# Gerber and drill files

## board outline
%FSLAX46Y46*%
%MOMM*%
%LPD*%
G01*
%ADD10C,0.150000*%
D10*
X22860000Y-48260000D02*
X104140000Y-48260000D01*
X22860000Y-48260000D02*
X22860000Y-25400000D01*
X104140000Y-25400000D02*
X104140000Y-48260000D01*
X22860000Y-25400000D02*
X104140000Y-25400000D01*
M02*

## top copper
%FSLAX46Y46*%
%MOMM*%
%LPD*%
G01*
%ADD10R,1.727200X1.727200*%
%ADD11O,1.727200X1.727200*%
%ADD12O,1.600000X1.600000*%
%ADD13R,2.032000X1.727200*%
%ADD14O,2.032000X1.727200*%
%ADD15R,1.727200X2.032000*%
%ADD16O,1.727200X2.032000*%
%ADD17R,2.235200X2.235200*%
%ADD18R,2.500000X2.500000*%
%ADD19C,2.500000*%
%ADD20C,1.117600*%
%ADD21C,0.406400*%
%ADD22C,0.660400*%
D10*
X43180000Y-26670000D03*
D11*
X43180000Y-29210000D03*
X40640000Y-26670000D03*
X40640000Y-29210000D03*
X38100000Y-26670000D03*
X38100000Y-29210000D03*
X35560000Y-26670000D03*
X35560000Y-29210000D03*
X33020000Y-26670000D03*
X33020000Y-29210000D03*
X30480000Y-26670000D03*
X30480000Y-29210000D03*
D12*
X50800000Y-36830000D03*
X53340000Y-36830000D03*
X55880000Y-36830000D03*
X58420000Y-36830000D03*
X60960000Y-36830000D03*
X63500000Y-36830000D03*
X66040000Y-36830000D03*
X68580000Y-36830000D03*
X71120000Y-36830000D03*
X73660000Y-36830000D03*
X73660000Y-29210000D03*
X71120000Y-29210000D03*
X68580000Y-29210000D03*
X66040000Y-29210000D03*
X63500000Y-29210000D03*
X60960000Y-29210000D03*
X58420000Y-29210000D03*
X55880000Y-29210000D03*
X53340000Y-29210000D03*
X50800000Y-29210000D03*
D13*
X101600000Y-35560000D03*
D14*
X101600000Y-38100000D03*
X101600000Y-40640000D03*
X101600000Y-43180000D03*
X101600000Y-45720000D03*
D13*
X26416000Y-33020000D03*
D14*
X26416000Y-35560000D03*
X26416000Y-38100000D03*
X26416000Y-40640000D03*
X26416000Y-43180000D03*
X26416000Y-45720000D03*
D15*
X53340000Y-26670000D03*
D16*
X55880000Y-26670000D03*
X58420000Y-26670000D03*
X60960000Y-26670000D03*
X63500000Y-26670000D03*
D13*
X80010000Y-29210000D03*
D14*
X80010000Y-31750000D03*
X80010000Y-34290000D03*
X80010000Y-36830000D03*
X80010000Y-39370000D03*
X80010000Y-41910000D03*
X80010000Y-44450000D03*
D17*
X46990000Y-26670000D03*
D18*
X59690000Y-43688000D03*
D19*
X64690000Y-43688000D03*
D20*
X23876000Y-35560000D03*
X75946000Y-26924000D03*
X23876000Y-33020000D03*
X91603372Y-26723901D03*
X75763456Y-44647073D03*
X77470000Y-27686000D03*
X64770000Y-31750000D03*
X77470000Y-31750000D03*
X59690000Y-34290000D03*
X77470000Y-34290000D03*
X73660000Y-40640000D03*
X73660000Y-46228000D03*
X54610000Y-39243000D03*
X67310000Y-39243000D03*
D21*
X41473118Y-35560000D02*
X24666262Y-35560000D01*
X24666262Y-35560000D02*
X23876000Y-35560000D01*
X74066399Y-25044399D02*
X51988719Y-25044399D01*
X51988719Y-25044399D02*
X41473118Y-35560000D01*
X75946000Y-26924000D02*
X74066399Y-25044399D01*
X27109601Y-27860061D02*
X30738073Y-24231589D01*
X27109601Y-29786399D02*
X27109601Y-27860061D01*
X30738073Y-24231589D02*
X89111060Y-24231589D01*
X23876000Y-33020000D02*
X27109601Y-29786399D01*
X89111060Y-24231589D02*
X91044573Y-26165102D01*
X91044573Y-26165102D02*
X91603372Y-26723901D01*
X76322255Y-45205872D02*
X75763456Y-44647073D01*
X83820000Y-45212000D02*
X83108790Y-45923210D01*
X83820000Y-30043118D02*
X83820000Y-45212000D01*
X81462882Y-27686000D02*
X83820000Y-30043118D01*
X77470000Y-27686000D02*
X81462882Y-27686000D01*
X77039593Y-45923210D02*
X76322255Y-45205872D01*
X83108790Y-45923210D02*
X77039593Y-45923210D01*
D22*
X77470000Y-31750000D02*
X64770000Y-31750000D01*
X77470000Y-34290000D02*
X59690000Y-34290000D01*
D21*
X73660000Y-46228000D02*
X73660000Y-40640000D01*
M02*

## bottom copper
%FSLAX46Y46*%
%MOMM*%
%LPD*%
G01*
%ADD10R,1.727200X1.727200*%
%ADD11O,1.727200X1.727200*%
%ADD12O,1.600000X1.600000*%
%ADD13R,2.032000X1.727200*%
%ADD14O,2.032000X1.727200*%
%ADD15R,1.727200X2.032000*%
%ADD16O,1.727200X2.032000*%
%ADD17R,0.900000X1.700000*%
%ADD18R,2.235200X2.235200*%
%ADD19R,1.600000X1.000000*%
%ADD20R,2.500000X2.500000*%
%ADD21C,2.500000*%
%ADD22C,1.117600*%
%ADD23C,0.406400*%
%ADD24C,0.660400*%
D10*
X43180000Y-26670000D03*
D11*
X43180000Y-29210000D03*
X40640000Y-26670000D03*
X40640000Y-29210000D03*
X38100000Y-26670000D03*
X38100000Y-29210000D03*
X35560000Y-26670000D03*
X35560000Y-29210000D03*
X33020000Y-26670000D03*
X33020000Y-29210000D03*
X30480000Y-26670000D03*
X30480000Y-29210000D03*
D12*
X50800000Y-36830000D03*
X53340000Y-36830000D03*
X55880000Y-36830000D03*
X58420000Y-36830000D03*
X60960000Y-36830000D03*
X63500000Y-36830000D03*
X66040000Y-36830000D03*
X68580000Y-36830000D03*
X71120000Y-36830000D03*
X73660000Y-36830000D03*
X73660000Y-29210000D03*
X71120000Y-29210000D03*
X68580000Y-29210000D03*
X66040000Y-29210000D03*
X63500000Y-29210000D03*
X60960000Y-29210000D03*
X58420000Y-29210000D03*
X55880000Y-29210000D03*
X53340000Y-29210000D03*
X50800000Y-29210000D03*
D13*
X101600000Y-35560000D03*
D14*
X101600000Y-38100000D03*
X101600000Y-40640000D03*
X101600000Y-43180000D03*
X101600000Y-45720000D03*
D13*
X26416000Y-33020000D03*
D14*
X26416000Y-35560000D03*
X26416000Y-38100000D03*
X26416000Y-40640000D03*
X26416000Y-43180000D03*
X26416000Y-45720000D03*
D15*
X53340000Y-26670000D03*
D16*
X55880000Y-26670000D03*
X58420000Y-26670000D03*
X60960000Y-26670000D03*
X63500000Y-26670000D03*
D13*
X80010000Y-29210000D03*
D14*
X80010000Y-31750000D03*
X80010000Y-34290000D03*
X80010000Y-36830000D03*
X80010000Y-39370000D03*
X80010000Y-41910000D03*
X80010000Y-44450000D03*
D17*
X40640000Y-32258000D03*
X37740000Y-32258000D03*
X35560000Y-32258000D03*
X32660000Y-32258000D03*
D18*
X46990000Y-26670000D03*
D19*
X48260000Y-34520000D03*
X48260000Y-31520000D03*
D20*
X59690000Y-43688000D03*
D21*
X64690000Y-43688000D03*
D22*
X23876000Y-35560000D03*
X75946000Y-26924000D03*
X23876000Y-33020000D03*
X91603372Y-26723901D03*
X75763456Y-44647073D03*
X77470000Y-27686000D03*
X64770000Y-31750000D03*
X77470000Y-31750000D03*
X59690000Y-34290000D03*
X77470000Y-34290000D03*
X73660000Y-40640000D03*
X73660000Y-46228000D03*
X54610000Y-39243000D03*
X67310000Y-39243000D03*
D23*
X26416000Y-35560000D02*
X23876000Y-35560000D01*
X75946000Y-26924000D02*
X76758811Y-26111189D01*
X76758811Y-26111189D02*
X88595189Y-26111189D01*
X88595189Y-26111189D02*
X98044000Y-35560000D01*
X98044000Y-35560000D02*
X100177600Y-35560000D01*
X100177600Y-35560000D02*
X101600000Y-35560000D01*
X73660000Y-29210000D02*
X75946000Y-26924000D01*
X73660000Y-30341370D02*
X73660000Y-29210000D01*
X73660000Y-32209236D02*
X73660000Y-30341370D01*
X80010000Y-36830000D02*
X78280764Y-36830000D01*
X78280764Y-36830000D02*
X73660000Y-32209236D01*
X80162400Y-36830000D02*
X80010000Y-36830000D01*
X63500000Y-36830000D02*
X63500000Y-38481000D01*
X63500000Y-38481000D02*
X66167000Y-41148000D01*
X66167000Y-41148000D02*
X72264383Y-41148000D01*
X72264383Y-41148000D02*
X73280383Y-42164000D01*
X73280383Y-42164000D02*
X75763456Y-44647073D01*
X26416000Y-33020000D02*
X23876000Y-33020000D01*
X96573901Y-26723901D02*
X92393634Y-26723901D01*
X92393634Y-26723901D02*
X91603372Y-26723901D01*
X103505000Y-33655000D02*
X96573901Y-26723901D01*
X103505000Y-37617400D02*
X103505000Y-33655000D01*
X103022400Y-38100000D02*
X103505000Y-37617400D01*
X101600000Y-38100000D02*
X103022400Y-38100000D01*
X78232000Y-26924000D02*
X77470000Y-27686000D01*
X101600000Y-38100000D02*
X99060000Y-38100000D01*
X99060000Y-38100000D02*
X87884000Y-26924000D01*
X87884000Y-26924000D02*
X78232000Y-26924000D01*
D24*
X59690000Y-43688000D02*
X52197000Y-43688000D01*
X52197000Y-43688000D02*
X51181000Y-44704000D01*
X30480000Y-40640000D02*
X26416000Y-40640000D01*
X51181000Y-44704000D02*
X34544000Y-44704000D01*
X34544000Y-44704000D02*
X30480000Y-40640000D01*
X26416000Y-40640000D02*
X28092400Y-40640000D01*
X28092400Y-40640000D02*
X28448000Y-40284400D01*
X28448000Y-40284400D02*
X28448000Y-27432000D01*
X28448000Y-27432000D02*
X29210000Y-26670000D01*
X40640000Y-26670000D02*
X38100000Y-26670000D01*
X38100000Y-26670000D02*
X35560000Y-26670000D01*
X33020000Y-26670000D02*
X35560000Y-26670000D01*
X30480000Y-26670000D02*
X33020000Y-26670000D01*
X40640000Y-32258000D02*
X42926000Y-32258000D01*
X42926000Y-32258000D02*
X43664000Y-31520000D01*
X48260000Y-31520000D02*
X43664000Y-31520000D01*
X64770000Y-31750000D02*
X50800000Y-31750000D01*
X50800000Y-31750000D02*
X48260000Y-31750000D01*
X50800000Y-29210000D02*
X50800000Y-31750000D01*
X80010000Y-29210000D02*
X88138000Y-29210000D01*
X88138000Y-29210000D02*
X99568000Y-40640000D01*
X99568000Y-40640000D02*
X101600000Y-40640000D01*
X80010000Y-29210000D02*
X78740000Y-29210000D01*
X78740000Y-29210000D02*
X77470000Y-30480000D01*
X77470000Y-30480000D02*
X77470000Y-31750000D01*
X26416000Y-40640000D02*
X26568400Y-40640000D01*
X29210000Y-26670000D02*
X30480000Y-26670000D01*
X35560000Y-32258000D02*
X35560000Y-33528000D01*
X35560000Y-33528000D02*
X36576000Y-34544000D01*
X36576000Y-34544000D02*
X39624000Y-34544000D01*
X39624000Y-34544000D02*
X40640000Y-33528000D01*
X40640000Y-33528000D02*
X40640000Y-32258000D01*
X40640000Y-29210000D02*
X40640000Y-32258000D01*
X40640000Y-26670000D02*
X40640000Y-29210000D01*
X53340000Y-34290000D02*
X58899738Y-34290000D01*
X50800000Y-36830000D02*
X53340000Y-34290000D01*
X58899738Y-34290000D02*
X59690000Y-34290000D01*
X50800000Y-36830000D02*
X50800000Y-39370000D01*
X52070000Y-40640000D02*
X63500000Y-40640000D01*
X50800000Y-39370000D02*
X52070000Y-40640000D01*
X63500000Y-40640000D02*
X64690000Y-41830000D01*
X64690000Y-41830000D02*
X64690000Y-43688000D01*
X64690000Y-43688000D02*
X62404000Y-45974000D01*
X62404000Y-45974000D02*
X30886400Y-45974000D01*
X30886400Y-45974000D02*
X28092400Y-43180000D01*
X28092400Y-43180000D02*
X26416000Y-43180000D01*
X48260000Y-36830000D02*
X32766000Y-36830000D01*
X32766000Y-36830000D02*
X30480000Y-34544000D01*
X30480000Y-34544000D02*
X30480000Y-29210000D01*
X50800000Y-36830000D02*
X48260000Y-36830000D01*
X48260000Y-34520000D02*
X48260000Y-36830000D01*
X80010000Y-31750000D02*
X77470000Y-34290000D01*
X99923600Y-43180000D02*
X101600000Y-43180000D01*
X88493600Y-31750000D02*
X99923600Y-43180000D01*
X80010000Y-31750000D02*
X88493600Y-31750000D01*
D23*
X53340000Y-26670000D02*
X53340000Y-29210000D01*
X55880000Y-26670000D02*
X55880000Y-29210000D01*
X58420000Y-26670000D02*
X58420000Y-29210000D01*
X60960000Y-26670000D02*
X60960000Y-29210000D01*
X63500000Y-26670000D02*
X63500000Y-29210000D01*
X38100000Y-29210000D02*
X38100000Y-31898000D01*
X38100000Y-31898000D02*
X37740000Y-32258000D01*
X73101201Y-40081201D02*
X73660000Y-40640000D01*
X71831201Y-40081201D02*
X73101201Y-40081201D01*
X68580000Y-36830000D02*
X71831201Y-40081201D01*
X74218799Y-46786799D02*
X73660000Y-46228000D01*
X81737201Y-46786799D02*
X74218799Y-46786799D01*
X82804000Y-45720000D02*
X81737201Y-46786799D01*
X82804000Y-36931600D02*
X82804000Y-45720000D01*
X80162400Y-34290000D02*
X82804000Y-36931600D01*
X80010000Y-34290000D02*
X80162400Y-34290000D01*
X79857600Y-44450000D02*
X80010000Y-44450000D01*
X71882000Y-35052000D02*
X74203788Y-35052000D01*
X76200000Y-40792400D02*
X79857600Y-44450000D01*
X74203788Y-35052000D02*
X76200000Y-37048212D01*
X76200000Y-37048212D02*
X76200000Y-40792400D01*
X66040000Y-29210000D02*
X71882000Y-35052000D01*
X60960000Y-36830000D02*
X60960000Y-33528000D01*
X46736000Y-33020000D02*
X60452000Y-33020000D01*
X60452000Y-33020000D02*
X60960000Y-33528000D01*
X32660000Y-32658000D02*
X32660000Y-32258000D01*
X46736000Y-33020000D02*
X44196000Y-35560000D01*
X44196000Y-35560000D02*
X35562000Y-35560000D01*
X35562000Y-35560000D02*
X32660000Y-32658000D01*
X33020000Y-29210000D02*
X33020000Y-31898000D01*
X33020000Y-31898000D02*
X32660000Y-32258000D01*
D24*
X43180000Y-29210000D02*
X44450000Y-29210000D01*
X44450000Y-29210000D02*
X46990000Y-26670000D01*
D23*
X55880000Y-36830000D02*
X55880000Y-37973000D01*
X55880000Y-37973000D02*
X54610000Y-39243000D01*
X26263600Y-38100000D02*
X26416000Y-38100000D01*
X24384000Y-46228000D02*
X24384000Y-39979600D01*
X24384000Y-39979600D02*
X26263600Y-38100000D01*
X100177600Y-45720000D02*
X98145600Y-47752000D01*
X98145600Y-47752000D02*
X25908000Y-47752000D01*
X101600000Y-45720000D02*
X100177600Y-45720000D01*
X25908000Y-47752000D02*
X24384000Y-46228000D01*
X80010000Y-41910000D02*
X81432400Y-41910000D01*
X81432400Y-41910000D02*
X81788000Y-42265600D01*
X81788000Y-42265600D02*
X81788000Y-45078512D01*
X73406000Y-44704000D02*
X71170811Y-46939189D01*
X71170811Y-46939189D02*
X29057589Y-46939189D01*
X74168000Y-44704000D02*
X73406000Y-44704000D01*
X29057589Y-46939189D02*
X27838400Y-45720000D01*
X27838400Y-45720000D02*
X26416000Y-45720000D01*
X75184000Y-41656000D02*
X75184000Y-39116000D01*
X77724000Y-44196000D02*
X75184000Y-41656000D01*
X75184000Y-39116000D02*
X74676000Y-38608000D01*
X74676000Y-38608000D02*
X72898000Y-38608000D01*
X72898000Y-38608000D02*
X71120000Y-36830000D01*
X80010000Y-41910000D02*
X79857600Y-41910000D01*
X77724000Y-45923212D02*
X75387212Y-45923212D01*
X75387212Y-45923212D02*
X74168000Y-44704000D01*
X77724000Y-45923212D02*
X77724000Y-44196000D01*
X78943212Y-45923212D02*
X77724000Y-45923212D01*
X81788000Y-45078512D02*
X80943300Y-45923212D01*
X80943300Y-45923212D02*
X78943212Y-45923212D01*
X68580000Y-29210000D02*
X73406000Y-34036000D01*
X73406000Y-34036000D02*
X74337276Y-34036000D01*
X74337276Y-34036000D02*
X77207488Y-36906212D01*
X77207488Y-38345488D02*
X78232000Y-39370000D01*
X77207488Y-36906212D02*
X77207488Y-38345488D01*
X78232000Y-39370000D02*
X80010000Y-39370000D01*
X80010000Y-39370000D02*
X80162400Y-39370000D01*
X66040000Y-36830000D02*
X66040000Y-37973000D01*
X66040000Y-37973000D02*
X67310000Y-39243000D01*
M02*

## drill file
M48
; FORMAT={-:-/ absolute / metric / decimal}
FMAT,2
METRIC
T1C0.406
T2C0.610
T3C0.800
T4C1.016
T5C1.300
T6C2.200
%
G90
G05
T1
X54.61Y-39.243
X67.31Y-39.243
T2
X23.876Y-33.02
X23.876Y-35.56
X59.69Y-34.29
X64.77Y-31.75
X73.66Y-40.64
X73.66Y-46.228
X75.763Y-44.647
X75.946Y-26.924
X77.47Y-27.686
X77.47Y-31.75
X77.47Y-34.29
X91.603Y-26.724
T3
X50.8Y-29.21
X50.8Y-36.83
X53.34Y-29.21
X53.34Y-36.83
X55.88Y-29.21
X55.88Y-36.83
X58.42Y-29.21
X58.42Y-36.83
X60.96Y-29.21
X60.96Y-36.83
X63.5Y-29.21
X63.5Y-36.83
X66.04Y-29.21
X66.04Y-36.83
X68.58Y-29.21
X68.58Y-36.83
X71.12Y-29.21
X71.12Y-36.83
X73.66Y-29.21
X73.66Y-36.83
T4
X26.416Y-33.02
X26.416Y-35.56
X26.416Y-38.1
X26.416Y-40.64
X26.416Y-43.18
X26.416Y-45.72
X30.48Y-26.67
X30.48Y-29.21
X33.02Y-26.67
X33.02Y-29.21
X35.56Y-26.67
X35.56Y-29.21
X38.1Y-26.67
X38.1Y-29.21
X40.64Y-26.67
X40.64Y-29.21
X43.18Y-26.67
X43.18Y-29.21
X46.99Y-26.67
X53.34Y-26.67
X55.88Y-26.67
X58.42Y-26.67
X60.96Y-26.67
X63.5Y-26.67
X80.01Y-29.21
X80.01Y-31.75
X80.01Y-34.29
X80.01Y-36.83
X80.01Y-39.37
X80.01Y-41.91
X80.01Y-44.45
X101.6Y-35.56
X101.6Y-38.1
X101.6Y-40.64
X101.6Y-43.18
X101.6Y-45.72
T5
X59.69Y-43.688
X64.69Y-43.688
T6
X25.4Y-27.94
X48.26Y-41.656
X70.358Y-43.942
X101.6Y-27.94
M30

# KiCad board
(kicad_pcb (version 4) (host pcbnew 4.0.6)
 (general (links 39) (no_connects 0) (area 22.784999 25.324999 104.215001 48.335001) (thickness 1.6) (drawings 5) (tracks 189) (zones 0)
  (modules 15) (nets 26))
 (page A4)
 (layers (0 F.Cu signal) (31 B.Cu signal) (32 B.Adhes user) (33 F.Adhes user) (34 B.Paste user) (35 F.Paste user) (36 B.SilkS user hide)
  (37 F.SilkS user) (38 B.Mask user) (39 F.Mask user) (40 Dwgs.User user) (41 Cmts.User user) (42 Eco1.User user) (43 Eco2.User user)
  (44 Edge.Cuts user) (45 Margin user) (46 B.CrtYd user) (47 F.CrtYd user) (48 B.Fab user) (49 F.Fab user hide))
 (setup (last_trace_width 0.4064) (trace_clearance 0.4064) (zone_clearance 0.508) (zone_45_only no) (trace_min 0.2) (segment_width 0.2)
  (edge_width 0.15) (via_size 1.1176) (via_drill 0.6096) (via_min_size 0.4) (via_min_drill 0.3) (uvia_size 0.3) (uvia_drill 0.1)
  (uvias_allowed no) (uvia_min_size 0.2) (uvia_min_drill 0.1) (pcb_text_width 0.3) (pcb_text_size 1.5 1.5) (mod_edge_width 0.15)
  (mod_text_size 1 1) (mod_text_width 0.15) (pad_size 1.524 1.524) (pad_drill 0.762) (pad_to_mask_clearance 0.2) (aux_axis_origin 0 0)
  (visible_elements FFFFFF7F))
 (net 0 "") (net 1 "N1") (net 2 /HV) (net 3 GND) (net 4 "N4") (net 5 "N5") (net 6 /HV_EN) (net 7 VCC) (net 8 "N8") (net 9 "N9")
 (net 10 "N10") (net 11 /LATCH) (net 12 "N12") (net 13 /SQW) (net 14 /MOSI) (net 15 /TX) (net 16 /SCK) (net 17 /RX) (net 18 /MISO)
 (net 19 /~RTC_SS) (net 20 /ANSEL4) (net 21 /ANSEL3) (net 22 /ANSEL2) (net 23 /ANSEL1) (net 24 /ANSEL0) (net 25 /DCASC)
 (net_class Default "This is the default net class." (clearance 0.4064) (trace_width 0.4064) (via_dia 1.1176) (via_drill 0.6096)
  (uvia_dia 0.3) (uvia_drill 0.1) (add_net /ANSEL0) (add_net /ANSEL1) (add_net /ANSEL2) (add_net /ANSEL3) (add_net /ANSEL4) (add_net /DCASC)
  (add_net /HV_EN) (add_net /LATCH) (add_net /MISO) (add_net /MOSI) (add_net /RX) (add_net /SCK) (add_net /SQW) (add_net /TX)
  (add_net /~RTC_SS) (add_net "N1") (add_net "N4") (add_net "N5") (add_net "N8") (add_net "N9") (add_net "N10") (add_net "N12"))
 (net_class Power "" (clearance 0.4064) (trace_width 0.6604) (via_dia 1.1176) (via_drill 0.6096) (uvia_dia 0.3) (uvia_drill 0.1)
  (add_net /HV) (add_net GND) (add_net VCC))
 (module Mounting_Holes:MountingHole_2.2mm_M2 (layer F.Cu) (at 70.358 43.942)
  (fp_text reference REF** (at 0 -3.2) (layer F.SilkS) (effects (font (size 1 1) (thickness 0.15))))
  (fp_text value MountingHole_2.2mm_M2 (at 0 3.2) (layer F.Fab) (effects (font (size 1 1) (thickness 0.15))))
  (pad 1 np_thru_hole circle (at 0 0) (size 2.2 2.2) (drill 2.2) (layers *.Cu *.Mask)))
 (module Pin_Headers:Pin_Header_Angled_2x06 (layer F.Cu) (at 43.18 26.67 270)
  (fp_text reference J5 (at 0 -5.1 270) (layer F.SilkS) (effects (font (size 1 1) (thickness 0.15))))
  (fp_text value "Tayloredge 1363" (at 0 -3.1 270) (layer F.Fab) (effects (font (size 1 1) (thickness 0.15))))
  (pad 1 thru_hole rect (at 0 0 270) (size 1.7272 1.7272) (drill 1.016) (layers *.Cu *.Mask) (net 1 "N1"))
  (pad 2 thru_hole oval (at 2.54 0 270) (size 1.7272 1.7272) (drill 1.016) (layers *.Cu *.Mask) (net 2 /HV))
  (pad 3 thru_hole oval (at 0 2.54 270) (size 1.7272 1.7272) (drill 1.016) (layers *.Cu *.Mask) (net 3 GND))
  (pad 4 thru_hole oval (at 2.54 2.54 270) (size 1.7272 1.7272) (drill 1.016) (layers *.Cu *.Mask) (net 3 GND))
  (pad 5 thru_hole oval (at 0 5.08 270) (size 1.7272 1.7272) (drill 1.016) (layers *.Cu *.Mask) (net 3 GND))
  (pad 6 thru_hole oval (at 2.54 5.08 270) (size 1.7272 1.7272) (drill 1.016) (layers *.Cu *.Mask) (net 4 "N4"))
  (pad 7 thru_hole oval (at 0 7.62 270) (size 1.7272 1.7272) (drill 1.016) (layers *.Cu *.Mask) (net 3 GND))
  (pad 8 thru_hole oval (at 2.54 7.62 270) (size 1.7272 1.7272) (drill 1.016) (layers *.Cu *.Mask) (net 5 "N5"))
  (pad 9 thru_hole oval (at 0 10.16 270) (size 1.7272 1.7272) (drill 1.016) (layers *.Cu *.Mask) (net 3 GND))
  (pad 10 thru_hole oval (at 2.54 10.16 270) (size 1.7272 1.7272) (drill 1.016) (layers *.Cu *.Mask) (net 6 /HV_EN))
  (pad 11 thru_hole oval (at 0 12.7 270) (size 1.7272 1.7272) (drill 1.016) (layers *.Cu *.Mask) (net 3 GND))
  (pad 12 thru_hole oval (at 2.54 12.7 270) (size 1.7272 1.7272) (drill 1.016) (layers *.Cu *.Mask) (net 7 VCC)))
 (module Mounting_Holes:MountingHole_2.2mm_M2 (layer F.Cu) (at 48.26 41.656)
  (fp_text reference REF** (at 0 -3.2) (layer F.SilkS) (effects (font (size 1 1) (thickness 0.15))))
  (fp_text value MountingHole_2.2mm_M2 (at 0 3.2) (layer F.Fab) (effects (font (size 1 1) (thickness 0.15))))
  (pad 1 np_thru_hole circle (at 0 0) (size 2.2 2.2) (drill 2.2) (layers *.Cu *.Mask)))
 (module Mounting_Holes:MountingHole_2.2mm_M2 (layer F.Cu) (at 25.4 27.94)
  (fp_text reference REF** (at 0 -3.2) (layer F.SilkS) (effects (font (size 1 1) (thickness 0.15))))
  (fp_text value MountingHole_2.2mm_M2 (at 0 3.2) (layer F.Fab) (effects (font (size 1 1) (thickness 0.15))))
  (pad 1 np_thru_hole circle (at 0 0) (size 2.2 2.2) (drill 2.2) (layers *.Cu *.Mask)))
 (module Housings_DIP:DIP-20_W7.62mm (layer F.Cu) (at 50.8 36.83 90)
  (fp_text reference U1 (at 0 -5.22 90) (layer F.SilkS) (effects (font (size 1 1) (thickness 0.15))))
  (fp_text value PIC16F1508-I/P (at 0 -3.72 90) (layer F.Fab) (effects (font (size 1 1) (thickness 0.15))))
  (pad 1 thru_hole oval (at 0 0 90) (size 1.6 1.6) (drill 0.8) (layers *.Cu *.Mask) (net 7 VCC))
  (pad 2 thru_hole oval (at 0 2.54 90) (size 1.6 1.6) (drill 0.8) (layers *.Cu *.Mask) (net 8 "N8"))
  (pad 3 thru_hole oval (at 0 5.08 90) (size 1.6 1.6) (drill 0.8) (layers *.Cu *.Mask) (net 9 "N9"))
  (pad 4 thru_hole oval (at 0 7.62 90) (size 1.6 1.6) (drill 0.8) (layers *.Cu *.Mask) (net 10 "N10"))
  (pad 5 thru_hole oval (at 0 10.16 90) (size 1.6 1.6) (drill 0.8) (layers *.Cu *.Mask) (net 6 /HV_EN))
  (pad 6 thru_hole oval (at 0 12.7 90) (size 1.6 1.6) (drill 0.8) (layers *.Cu *.Mask) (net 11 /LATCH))
  (pad 7 thru_hole oval (at 0 15.24 90) (size 1.6 1.6) (drill 0.8) (layers *.Cu *.Mask) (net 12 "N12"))
  (pad 8 thru_hole oval (at 0 17.78 90) (size 1.6 1.6) (drill 0.8) (layers *.Cu *.Mask) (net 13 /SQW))
  (pad 9 thru_hole oval (at 0 20.32 90) (size 1.6 1.6) (drill 0.8) (layers *.Cu *.Mask) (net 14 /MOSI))
  (pad 10 thru_hole oval (at 0 22.86 90) (size 1.6 1.6) (drill 0.8) (layers *.Cu *.Mask) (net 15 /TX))
  (pad 11 thru_hole oval (at 7.62 22.86 90) (size 1.6 1.6) (drill 0.8) (layers *.Cu *.Mask) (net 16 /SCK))
  (pad 12 thru_hole oval (at 7.62 20.32 90) (size 1.6 1.6) (drill 0.8) (layers *.Cu *.Mask) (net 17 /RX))
  (pad 13 thru_hole oval (at 7.62 17.78 90) (size 1.6 1.6) (drill 0.8) (layers *.Cu *.Mask) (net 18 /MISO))
  (pad 14 thru_hole oval (at 7.62 15.24 90) (size 1.6 1.6) (drill 0.8) (layers *.Cu *.Mask) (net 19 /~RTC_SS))
  (pad 15 thru_hole oval (at 7.62 12.7 90) (size 1.6 1.6) (drill 0.8) (layers *.Cu *.Mask) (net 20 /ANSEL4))
  (pad 16 thru_hole oval (at 7.62 10.16 90) (size 1.6 1.6) (drill 0.8) (layers *.Cu *.Mask) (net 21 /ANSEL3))
  (pad 17 thru_hole oval (at 7.62 7.62 90) (size 1.6 1.6) (drill 0.8) (layers *.Cu *.Mask) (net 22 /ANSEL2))
  (pad 18 thru_hole oval (at 7.62 5.08 90) (size 1.6 1.6) (drill 0.8) (layers *.Cu *.Mask) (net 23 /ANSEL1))
  (pad 19 thru_hole oval (at 7.62 2.54 90) (size 1.6 1.6) (drill 0.8) (layers *.Cu *.Mask) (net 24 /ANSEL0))
  (pad 20 thru_hole oval (at 7.62 0 90) (size 1.6 1.6) (drill 0.8) (layers *.Cu *.Mask) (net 3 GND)))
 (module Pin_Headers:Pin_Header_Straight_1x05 (layer F.Cu) (at 101.6 35.56)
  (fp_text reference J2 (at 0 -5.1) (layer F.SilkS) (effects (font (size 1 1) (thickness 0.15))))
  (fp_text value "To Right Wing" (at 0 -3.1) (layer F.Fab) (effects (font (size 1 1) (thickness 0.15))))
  (pad 1 thru_hole rect (at 0 0) (size 2.032 1.7272) (drill 1.016) (layers *.Cu *.Mask) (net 16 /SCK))
  (pad 2 thru_hole oval (at 0 2.54) (size 2.032 1.7272) (drill 1.016) (layers *.Cu *.Mask) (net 11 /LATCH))
  (pad 3 thru_hole oval (at 0 5.08) (size 2.032 1.7272) (drill 1.016) (layers *.Cu *.Mask) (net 3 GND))
  (pad 4 thru_hole oval (at 0 7.62) (size 2.032 1.7272) (drill 1.016) (layers *.Cu *.Mask) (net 7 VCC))
  (pad 5 thru_hole oval (at 0 10.16) (size 2.032 1.7272) (drill 1.016) (layers *.Cu *.Mask) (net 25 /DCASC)))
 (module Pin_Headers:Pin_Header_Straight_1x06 (layer F.Cu) (at 26.416 33.02)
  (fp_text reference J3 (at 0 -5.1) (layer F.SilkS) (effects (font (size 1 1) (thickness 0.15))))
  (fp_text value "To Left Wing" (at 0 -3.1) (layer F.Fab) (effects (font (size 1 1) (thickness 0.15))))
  (pad 1 thru_hole rect (at 0 0) (size 2.032 1.7272) (drill 1.016) (layers *.Cu *.Mask) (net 11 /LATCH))
  (pad 2 thru_hole oval (at 0 2.54) (size 2.032 1.7272) (drill 1.016) (layers *.Cu *.Mask) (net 16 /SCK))
  (pad 3 thru_hole oval (at 0 5.08) (size 2.032 1.7272) (drill 1.016) (layers *.Cu *.Mask) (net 25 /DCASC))
  (pad 4 thru_hole oval (at 0 7.62) (size 2.032 1.7272) (drill 1.016) (layers *.Cu *.Mask) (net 3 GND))
  (pad 5 thru_hole oval (at 0 10.16) (size 2.032 1.7272) (drill 1.016) (layers *.Cu *.Mask) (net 7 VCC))
  (pad 6 thru_hole oval (at 0 12.7) (size 2.032 1.7272) (drill 1.016) (layers *.Cu *.Mask) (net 14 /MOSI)))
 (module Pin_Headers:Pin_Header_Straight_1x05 (layer F.Cu) (at 53.34 26.67 90)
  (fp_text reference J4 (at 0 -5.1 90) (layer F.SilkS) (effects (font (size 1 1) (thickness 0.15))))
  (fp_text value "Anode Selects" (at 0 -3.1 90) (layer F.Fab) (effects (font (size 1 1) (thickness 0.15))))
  (pad 1 thru_hole rect (at 0 0 90) (size 2.032 1.7272) (drill 1.016) (layers *.Cu *.Mask) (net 24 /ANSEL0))
  (pad 2 thru_hole oval (at 0 2.54 90) (size 2.032 1.7272) (drill 1.016) (layers *.Cu *.Mask) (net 23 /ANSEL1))
  (pad 3 thru_hole oval (at 0 5.08 90) (size 2.032 1.7272) (drill 1.016) (layers *.Cu *.Mask) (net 22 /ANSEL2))
  (pad 4 thru_hole oval (at 0 7.62 90) (size 2.032 1.7272) (drill 1.016) (layers *.Cu *.Mask) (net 21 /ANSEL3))
  (pad 5 thru_hole oval (at 0 10.16 90) (size 2.032 1.7272) (drill 1.016) (layers *.Cu *.Mask) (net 20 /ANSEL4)))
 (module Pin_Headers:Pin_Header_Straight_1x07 (layer F.Cu) (at 80.01 29.21)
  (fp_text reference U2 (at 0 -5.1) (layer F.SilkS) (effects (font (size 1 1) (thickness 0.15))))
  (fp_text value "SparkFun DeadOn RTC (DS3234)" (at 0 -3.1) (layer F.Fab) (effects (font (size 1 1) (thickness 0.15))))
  (pad 1 thru_hole rect (at 0 0) (size 2.032 1.7272) (drill 1.016) (layers *.Cu *.Mask) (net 3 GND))
  (pad 2 thru_hole oval (at 0 2.54) (size 2.032 1.7272) (drill 1.016) (layers *.Cu *.Mask) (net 7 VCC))
  (pad 3 thru_hole oval (at 0 5.08) (size 2.032 1.7272) (drill 1.016) (layers *.Cu *.Mask) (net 13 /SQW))
  (pad 4 thru_hole oval (at 0 7.62) (size 2.032 1.7272) (drill 1.016) (layers *.Cu *.Mask) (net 16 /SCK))
  (pad 5 thru_hole oval (at 0 10.16) (size 2.032 1.7272) (drill 1.016) (layers *.Cu *.Mask) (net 18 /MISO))
  (pad 6 thru_hole oval (at 0 12.7) (size 2.032 1.7272) (drill 1.016) (layers *.Cu *.Mask) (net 14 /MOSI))
  (pad 7 thru_hole oval (at 0 15.24) (size 2.032 1.7272) (drill 1.016) (layers *.Cu *.Mask) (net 19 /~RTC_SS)))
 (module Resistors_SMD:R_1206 (layer B.Cu) (at 39.19 32.258 180)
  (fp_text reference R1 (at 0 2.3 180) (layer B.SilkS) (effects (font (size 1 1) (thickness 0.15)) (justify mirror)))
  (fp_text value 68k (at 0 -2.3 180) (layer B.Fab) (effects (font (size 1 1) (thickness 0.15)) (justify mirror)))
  (pad 1 smd rect (at -1.45 0 180) (size 0.9 1.7) (layers B.Cu B.Paste B.Mask) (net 3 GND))
  (pad 2 smd rect (at 1.45 0 180) (size 0.9 1.7) (layers B.Cu B.Paste B.Mask) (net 4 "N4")))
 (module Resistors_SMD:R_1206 (layer B.Cu) (at 34.11 32.258 180)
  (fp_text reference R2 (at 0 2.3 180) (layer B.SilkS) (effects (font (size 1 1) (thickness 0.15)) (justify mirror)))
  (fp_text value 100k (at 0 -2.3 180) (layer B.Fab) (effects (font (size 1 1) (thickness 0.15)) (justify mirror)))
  (pad 1 smd rect (at -1.45 0 180) (size 0.9 1.7) (layers B.Cu B.Paste B.Mask) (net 3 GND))
  (pad 2 smd rect (at 1.45 0 180) (size 0.9 1.7) (layers B.Cu B.Paste B.Mask) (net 6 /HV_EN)))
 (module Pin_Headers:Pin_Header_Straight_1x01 (layer F.Cu) (at 46.99 26.67 180)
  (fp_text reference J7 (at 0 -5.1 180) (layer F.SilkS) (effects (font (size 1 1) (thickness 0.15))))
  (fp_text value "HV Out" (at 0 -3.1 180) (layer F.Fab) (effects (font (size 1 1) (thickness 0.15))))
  (pad 1 thru_hole rect (at 0 0 180) (size 2.2352 2.2352) (drill 1.016) (layers *.Cu *.Mask) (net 2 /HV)))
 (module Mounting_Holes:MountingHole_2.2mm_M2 (layer F.Cu) (at 101.6 27.94)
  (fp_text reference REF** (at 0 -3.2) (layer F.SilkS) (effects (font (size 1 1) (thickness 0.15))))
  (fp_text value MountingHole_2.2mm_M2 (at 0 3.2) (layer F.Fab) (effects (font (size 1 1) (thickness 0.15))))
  (pad 1 np_thru_hole circle (at 0 0) (size 2.2 2.2) (drill 2.2) (layers *.Cu *.Mask)))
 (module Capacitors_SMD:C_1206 (layer B.Cu) (at 48.26 33.02 90)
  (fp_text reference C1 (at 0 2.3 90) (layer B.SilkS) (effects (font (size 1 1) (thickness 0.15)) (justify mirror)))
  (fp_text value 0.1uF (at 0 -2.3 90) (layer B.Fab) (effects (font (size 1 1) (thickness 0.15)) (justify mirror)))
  (pad 1 smd rect (at -1.5 0 90) (size 1 1.6) (layers B.Cu B.Paste B.Mask) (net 7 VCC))
  (pad 2 smd rect (at 1.5 0 90) (size 1 1.6) (layers B.Cu B.Paste B.Mask) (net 3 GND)))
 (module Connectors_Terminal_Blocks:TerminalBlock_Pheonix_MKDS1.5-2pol (layer F.Cu) (at 59.69 43.688)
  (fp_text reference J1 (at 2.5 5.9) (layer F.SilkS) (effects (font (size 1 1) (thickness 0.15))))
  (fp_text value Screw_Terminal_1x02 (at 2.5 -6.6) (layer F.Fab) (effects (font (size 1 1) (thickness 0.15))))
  (pad 1 thru_hole rect (at 0 0) (size 2.5 2.5) (drill 1.3) (layers *.Cu *.Mask) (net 3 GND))
  (pad 2 thru_hole circle (at 5 0) (size 2.5 2.5) (drill 1.3) (layers *.Cu *.Mask) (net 7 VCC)))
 (gr_line (start 22.86 48.26) (end 104.14 48.26) (layer Edge.Cuts) (width 0.15))
 (gr_line (start 22.86 48.26) (end 22.86 25.4) (layer Edge.Cuts) (width 0.15))
 (gr_line (start 104.14 25.4) (end 104.14 48.26) (layer Edge.Cuts) (width 0.15))
 (gr_line (start 22.86 25.4) (end 104.14 25.4) (layer Edge.Cuts) (width 0.15))
 (segment (start 26.416 35.56) (end 23.876 35.56) (width 0.4064) (layer B.Cu) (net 16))
 (segment (start 41.473118 35.56) (end 24.666262 35.56) (width 0.4064) (layer F.Cu) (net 16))
 (segment (start 24.666262 35.56) (end 23.876 35.56) (width 0.4064) (layer F.Cu) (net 16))
 (via (at 23.876 35.56) (size 1.1176) (drill 0.6096) (layers F.Cu B.Cu) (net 16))
 (segment (start 74.066399 25.044399) (end 51.988719 25.044399) (width 0.4064) (layer F.Cu) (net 16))
 (segment (start 51.988719 25.044399) (end 41.473118 35.56) (width 0.4064) (layer F.Cu) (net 16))
 (segment (start 75.946 26.924) (end 74.066399 25.044399) (width 0.4064) (layer F.Cu) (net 16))
 (segment (start 75.946 26.924) (end 76.758811 26.111189) (width 0.4064) (layer B.Cu) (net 16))
 (segment (start 76.758811 26.111189) (end 88.595189 26.111189) (width 0.4064) (layer B.Cu) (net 16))
 (segment (start 88.595189 26.111189) (end 98.044 35.56) (width 0.4064) (layer B.Cu) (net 16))
 (segment (start 98.044 35.56) (end 100.1776 35.56) (width 0.4064) (layer B.Cu) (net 16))
 (segment (start 100.1776 35.56) (end 101.6 35.56) (width 0.4064) (layer B.Cu) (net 16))
 (segment (start 73.66 29.21) (end 75.946 26.924) (width 0.4064) (layer B.Cu) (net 16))
 (via (at 75.946 26.924) (size 1.1176) (drill 0.6096) (layers F.Cu B.Cu) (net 16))
 (segment (start 73.66 30.34137) (end 73.66 29.21) (width 0.4064) (layer B.Cu) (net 16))
 (segment (start 73.66 32.209236) (end 73.66 30.34137) (width 0.4064) (layer B.Cu) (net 16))
 (segment (start 80.01 36.83) (end 78.280764 36.83) (width 0.4064) (layer B.Cu) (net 16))
 (segment (start 78.280764 36.83) (end 73.66 32.209236) (width 0.4064) (layer B.Cu) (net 16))
 (segment (start 80.1624 36.83) (end 80.01 36.83) (width 0.4064) (layer B.Cu) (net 16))
 (segment (start 63.5 36.83) (end 63.5 38.481) (width 0.4064) (layer B.Cu) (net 11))
 (segment (start 63.5 38.481) (end 66.167 41.148) (width 0.4064) (layer B.Cu) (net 11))
 (segment (start 66.167 41.148) (end 72.264383 41.148) (width 0.4064) (layer B.Cu) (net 11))
 (segment (start 72.264383 41.148) (end 73.280383 42.164) (width 0.4064) (layer B.Cu) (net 11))
 (segment (start 73.280383 42.164) (end 75.763456 44.647073) (width 0.4064) (layer B.Cu) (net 11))
 (segment (start 27.109601 27.860061) (end 30.738073 24.231589) (width 0.4064) (layer F.Cu) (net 11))
 (segment (start 27.109601 29.786399) (end 27.109601 27.860061) (width 0.4064) (layer F.Cu) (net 11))
 (segment (start 30.738073 24.231589) (end 89.11106 24.231589) (width 0.4064) (layer F.Cu) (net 11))
 (segment (start 23.876 33.02) (end 27.109601 29.786399) (width 0.4064) (layer F.Cu) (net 11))
 (via (at 23.876 33.02) (size 1.1176) (drill 0.6096) (layers F.Cu B.Cu) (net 11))
 (segment (start 26.416 33.02) (end 23.876 33.02) (width 0.4064) (layer B.Cu) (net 11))
 (segment (start 89.11106 24.231589) (end 91.044573 26.165102) (width 0.4064) (layer F.Cu) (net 11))
 (segment (start 91.044573 26.165102) (end 91.603372 26.723901) (width 0.4064) (layer F.Cu) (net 11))
 (via (at 91.603372 26.723901) (size 1.1176) (drill 0.6096) (layers F.Cu B.Cu) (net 11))
 (segment (start 96.573901 26.723901) (end 92.393634 26.723901) (width 0.4064) (layer B.Cu) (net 11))
 (segment (start 92.393634 26.723901) (end 91.603372 26.723901) (width 0.4064) (layer B.Cu) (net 11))
 (segment (start 103.505 33.655) (end 96.573901 26.723901) (width 0.4064) (layer B.Cu) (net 11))
 (segment (start 103.505 37.6174) (end 103.505 33.655) (width 0.4064) (layer B.Cu) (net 11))
 (segment (start 103.0224 38.1) (end 103.505 37.6174) (width 0.4064) (layer B.Cu) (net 11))
 (segment (start 101.6 38.1) (end 103.0224 38.1) (width 0.4064) (layer B.Cu) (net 11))
 (segment (start 76.322255 45.205872) (end 75.763456 44.647073) (width 0.4064) (layer F.Cu) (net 11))
 (segment (start 83.82 45.212) (end 83.10879 45.92321) (width 0.4064) (layer F.Cu) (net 11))
 (segment (start 83.82 30.043118) (end 83.82 45.212) (width 0.4064) (layer F.Cu) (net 11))
 (segment (start 81.462882 27.686) (end 83.82 30.043118) (width 0.4064) (layer F.Cu) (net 11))
 (segment (start 77.47 27.686) (end 81.462882 27.686) (width 0.4064) (layer F.Cu) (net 11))
 (segment (start 77.039593 45.92321) (end 76.322255 45.205872) (width 0.4064) (layer F.Cu) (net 11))
 (segment (start 83.10879 45.92321) (end 77.039593 45.92321) (width 0.4064) (layer F.Cu) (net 11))
 (via (at 75.763456 44.647073) (size 1.1176) (drill 0.6096) (layers F.Cu B.Cu) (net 11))
 (segment (start 78.232 26.924) (end 77.47 27.686) (width 0.4064) (layer B.Cu) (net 11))
 (via (at 77.47 27.686) (size 1.1176) (drill 0.6096) (layers F.Cu B.Cu) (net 11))
 (segment (start 101.6 38.1) (end 99.06 38.1) (width 0.4064) (layer B.Cu) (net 11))
 (segment (start 99.06 38.1) (end 87.884 26.924) (width 0.4064) (layer B.Cu) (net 11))
 (segment (start 87.884 26.924) (end 78.232 26.924) (width 0.4064) (layer B.Cu) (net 11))
 (segment (start 59.69 43.688) (end 52.197 43.688) (width 0.6604) (layer B.Cu) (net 3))
 (segment (start 52.197 43.688) (end 51.181 44.704) (width 0.6604) (layer B.Cu) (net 3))
 (segment (start 30.48 40.64) (end 26.416 40.64) (width 0.6604) (layer B.Cu) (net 3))
 (segment (start 51.181 44.704) (end 34.544 44.704) (width 0.6604) (layer B.Cu) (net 3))
 (segment (start 34.544 44.704) (end 30.48 40.64) (width 0.6604) (layer B.Cu) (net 3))
 (segment (start 26.416 40.64) (end 28.0924 40.64) (width 0.6604) (layer B.Cu) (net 3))
 (segment (start 28.0924 40.64) (end 28.448 40.2844) (width 0.6604) (layer B.Cu) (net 3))
 (segment (start 28.448 40.2844) (end 28.448 27.432) (width 0.6604) (layer B.Cu) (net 3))
 (segment (start 28.448 27.432) (end 29.21 26.67) (width 0.6604) (layer B.Cu) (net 3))
 (segment (start 40.64 26.67) (end 38.1 26.67) (width 0.6604) (layer B.Cu) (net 3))
 (segment (start 38.1 26.67) (end 35.56 26.67) (width 0.6604) (layer B.Cu) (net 3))
 (segment (start 33.02 26.67) (end 35.56 26.67) (width 0.6604) (layer B.Cu) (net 3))
 (segment (start 30.48 26.67) (end 33.02 26.67) (width 0.6604) (layer B.Cu) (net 3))
 (segment (start 40.64 32.258) (end 42.926 32.258) (width 0.6604) (layer B.Cu) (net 3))
 (segment (start 42.926 32.258) (end 43.664 31.52) (width 0.6604) (layer B.Cu) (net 3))
 (segment (start 48.26 31.52) (end 43.664 31.52) (width 0.6604) (layer B.Cu) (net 3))
 (segment (start 64.77 31.75) (end 50.8 31.75) (width 0.6604) (layer B.Cu) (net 3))
 (segment (start 50.8 31.75) (end 48.26 31.75) (width 0.6604) (layer B.Cu) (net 3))
 (segment (start 50.8 29.21) (end 50.8 31.75) (width 0.6604) (layer B.Cu) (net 3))
 (segment (start 80.01 29.21) (end 88.138 29.21) (width 0.6604) (layer B.Cu) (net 3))
 (segment (start 88.138 29.21) (end 99.568 40.64) (width 0.6604) (layer B.Cu) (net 3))
 (segment (start 99.568 40.64) (end 101.6 40.64) (width 0.6604) (layer B.Cu) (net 3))
 (segment (start 80.01 29.21) (end 78.74 29.21) (width 0.6604) (layer B.Cu) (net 3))
 (segment (start 78.74 29.21) (end 77.47 30.48) (width 0.6604) (layer B.Cu) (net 3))
 (segment (start 77.47 30.48) (end 77.47 31.75) (width 0.6604) (layer B.Cu) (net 3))
 (segment (start 26.416 40.64) (end 26.5684 40.64) (width 0.6604) (layer B.Cu) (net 3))
 (segment (start 29.21 26.67) (end 30.48 26.67) (width 0.6604) (layer B.Cu) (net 3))
 (segment (start 35.56 32.258) (end 35.56 33.528) (width 0.6604) (layer B.Cu) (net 3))
 (segment (start 35.56 33.528) (end 36.576 34.544) (width 0.6604) (layer B.Cu) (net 3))
 (segment (start 36.576 34.544) (end 39.624 34.544) (width 0.6604) (layer B.Cu) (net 3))
 (segment (start 39.624 34.544) (end 40.64 33.528) (width 0.6604) (layer B.Cu) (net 3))
 (segment (start 40.64 33.528) (end 40.64 32.258) (width 0.6604) (layer B.Cu) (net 3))
 (segment (start 40.64 29.21) (end 40.64 32.258) (width 0.6604) (layer B.Cu) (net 3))
 (segment (start 40.64 26.67) (end 40.64 29.21) (width 0.6604) (layer B.Cu) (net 3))
 (via (at 64.77 31.75) (size 1.1176) (drill 0.6096) (layers F.Cu B.Cu) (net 3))
 (segment (start 77.47 31.75) (end 64.77 31.75) (width 0.6604) (layer F.Cu) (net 3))
 (via (at 77.47 31.75) (size 1.1176) (drill 0.6096) (layers F.Cu B.Cu) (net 3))
 (segment (start 53.34 34.29) (end 58.899738 34.29) (width 0.6604) (layer B.Cu) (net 7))
 (segment (start 50.8 36.83) (end 53.34 34.29) (width 0.6604) (layer B.Cu) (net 7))
 (segment (start 58.899738 34.29) (end 59.69 34.29) (width 0.6604) (layer B.Cu) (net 7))
 (segment (start 77.47 34.29) (end 59.69 34.29) (width 0.6604) (layer F.Cu) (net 7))
 (via (at 59.69 34.29) (size 1.1176) (drill 0.6096) (layers F.Cu B.Cu) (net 7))
 (segment (start 50.8 36.83) (end 50.8 39.37) (width 0.6604) (layer B.Cu) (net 7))
 (segment (start 52.07 40.64) (end 63.5 40.64) (width 0.6604) (layer B.Cu) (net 7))
 (segment (start 50.8 39.37) (end 52.07 40.64) (width 0.6604) (layer B.Cu) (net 7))
 (segment (start 63.5 40.64) (end 64.69 41.83) (width 0.6604) (layer B.Cu) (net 7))
 (segment (start 64.69 41.83) (end 64.69 43.688) (width 0.6604) (layer B.Cu) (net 7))
 (segment (start 64.69 43.688) (end 62.404 45.974) (width 0.6604) (layer B.Cu) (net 7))
 (segment (start 62.404 45.974) (end 30.8864 45.974) (width 0.6604) (layer B.Cu) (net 7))
 (segment (start 30.8864 45.974) (end 28.0924 43.18) (width 0.6604) (layer B.Cu) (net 7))
 (segment (start 28.0924 43.18) (end 26.416 43.18) (width 0.6604) (layer B.Cu) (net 7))
 (segment (start 48.26 36.83) (end 32.766 36.83) (width 0.6604) (layer B.Cu) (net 7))
 (segment (start 32.766 36.83) (end 30.48 34.544) (width 0.6604) (layer B.Cu) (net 7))
 (segment (start 30.48 34.544) (end 30.48 29.21) (width 0.6604) (layer B.Cu) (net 7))
 (segment (start 50.8 36.83) (end 48.26 36.83) (width 0.6604) (layer B.Cu) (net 7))
 (segment (start 48.26 34.52) (end 48.26 36.83) (width 0.6604) (layer B.Cu) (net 7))
 (segment (start 80.01 31.75) (end 77.47 34.29) (width 0.6604) (layer B.Cu) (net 7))
 (via (at 77.47 34.29) (size 1.1176) (drill 0.6096) (layers F.Cu B.Cu) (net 7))
 (segment (start 99.9236 43.18) (end 101.6 43.18) (width 0.6604) (layer B.Cu) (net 7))
 (segment (start 88.4936 31.75) (end 99.9236 43.18) (width 0.6604) (layer B.Cu) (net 7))
 (segment (start 80.01 31.75) (end 88.4936 31.75) (width 0.6604) (layer B.Cu) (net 7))
 (segment (start 53.34 26.67) (end 53.34 29.21) (width 0.4064) (layer B.Cu) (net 24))
 (segment (start 55.88 26.67) (end 55.88 29.21) (width 0.4064) (layer B.Cu) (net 23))
 (segment (start 58.42 26.67) (end 58.42 29.21) (width 0.4064) (layer B.Cu) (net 22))
 (segment (start 60.96 26.67) (end 60.96 29.21) (width 0.4064) (layer B.Cu) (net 21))
 (segment (start 63.5 26.67) (end 63.5 29.21) (width 0.4064) (layer B.Cu) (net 20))
 (segment (start 38.1 29.21) (end 38.1 31.898) (width 0.4064) (layer B.Cu) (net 4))
 (segment (start 38.1 31.898) (end 37.74 32.258) (width 0.4064) (layer B.Cu) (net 4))
 (segment (start 73.101201 40.081201) (end 73.66 40.64) (width 0.4064) (layer B.Cu) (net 13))
 (segment (start 71.831201 40.081201) (end 73.101201 40.081201) (width 0.4064) (layer B.Cu) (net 13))
 (segment (start 68.58 36.83) (end 71.831201 40.081201) (width 0.4064) (layer B.Cu) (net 13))
 (segment (start 73.66 46.228) (end 73.66 40.64) (width 0.4064) (layer F.Cu) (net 13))
 (via (at 73.66 40.64) (size 1.1176) (drill 0.6096) (layers F.Cu B.Cu) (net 13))
 (segment (start 74.218799 46.786799) (end 73.66 46.228) (width 0.4064) (layer B.Cu) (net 13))
 (segment (start 81.737201 46.786799) (end 74.218799 46.786799) (width 0.4064) (layer B.Cu) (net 13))
 (segment (start 82.804 45.72) (end 81.737201 46.786799) (width 0.4064) (layer B.Cu) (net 13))
 (segment (start 82.804 36.9316) (end 82.804 45.72) (width 0.4064) (layer B.Cu) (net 13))
 (segment (start 80.1624 34.29) (end 82.804 36.9316) (width 0.4064) (layer B.Cu) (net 13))
 (segment (start 80.01 34.29) (end 80.1624 34.29) (width 0.4064) (layer B.Cu) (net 13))
 (via (at 73.66 46.228) (size 1.1176) (drill 0.6096) (layers F.Cu B.Cu) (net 13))
 (segment (start 79.8576 44.45) (end 80.01 44.45) (width 0.4064) (layer B.Cu) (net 19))
 (segment (start 71.882 35.052) (end 74.203788 35.052) (width 0.4064) (layer B.Cu) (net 19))
 (segment (start 76.2 40.7924) (end 79.8576 44.45) (width 0.4064) (layer B.Cu) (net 19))
 (segment (start 74.203788 35.052) (end 76.2 37.048212) (width 0.4064) (layer B.Cu) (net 19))
 (segment (start 76.2 37.048212) (end 76.2 40.7924) (width 0.4064) (layer B.Cu) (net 19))
 (segment (start 66.04 29.21) (end 71.882 35.052) (width 0.4064) (layer B.Cu) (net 19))
 (segment (start 60.96 36.83) (end 60.96 33.528) (width 0.4064) (layer B.Cu) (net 6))
 (segment (start 46.736 33.02) (end 60.452 33.02) (width 0.4064) (layer B.Cu) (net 6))
 (segment (start 60.452 33.02) (end 60.96 33.528) (width 0.4064) (layer B.Cu) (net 6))
 (segment (start 32.66 32.658) (end 32.66 32.258) (width 0.4064) (layer B.Cu) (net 6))
 (segment (start 46.736 33.02) (end 44.196 35.56) (width 0.4064) (layer B.Cu) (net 6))
 (segment (start 44.196 35.56) (end 35.562 35.56) (width 0.4064) (layer B.Cu) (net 6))
 (segment (start 35.562 35.56) (end 32.66 32.658) (width 0.4064) (layer B.Cu) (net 6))
 (segment (start 33.02 29.21) (end 33.02 31.898) (width 0.4064) (layer B.Cu) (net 6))
 (segment (start 33.02 31.898) (end 32.66 32.258) (width 0.4064) (layer B.Cu) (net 6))
 (segment (start 43.18 29.21) (end 44.45 29.21) (width 0.6604) (layer B.Cu) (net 2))
 (segment (start 44.45 29.21) (end 46.99 26.67) (width 0.6604) (layer B.Cu) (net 2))
 (segment (start 55.88 36.83) (end 55.88 37.973) (width 0.4064) (layer B.Cu) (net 9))
 (segment (start 55.88 37.973) (end 54.61 39.243) (width 0.4064) (layer B.Cu) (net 9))
 (via (at 54.61 39.243) (size 1.1176) (drill 0.4064) (layers F.Cu B.Cu) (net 9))
 (segment (start 26.2636 38.1) (end 26.416 38.1) (width 0.4064) (layer B.Cu) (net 25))
 (segment (start 24.384 46.228) (end 24.384 39.9796) (width 0.4064) (layer B.Cu) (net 25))
 (segment (start 24.384 39.9796) (end 26.2636 38.1) (width 0.4064) (layer B.Cu) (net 25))
 (segment (start 100.1776 45.72) (end 98.1456 47.752) (width 0.4064) (layer B.Cu) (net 25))
 (segment (start 98.1456 47.752) (end 25.908 47.752) (width 0.4064) (layer B.Cu) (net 25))
 (segment (start 101.6 45.72) (end 100.1776 45.72) (width 0.4064) (layer B.Cu) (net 25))
 (segment (start 25.908 47.752) (end 24.384 46.228) (width 0.4064) (layer B.Cu) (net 25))
 (segment (start 80.01 41.91) (end 81.4324 41.91) (width 0.4064) (layer B.Cu) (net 14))
 (segment (start 81.4324 41.91) (end 81.788 42.2656) (width 0.4064) (layer B.Cu) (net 14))
 (segment (start 81.788 42.2656) (end 81.788 45.078512) (width 0.4064) (layer B.Cu) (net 14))
 (segment (start 73.406 44.704) (end 71.170811 46.939189) (width 0.4064) (layer B.Cu) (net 14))
 (segment (start 71.170811 46.939189) (end 29.057589 46.939189) (width 0.4064) (layer B.Cu) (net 14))
 (segment (start 74.168 44.704) (end 73.406 44.704) (width 0.4064) (layer B.Cu) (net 14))
 (segment (start 29.057589 46.939189) (end 27.8384 45.72) (width 0.4064) (layer B.Cu) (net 14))
 (segment (start 27.8384 45.72) (end 26.416 45.72) (width 0.4064) (layer B.Cu) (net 14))
 (segment (start 75.184 41.656) (end 75.184 39.116) (width 0.4064) (layer B.Cu) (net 14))
 (segment (start 77.724 44.196) (end 75.184 41.656) (width 0.4064) (layer B.Cu) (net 14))
 (segment (start 75.184 39.116) (end 74.676 38.608) (width 0.4064) (layer B.Cu) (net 14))
 (segment (start 74.676 38.608) (end 72.898 38.608) (width 0.4064) (layer B.Cu) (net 14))
 (segment (start 72.898 38.608) (end 71.12 36.83) (width 0.4064) (layer B.Cu) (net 14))
 (segment (start 80.01 41.91) (end 79.8576 41.91) (width 0.4064) (layer B.Cu) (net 14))
 (segment (start 77.724 45.923212) (end 75.387212 45.923212) (width 0.4064) (layer B.Cu) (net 14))
 (segment (start 75.387212 45.923212) (end 74.168 44.704) (width 0.4064) (layer B.Cu) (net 14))
 (segment (start 77.724 45.923212) (end 77.724 44.196) (width 0.4064) (layer B.Cu) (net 14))
 (segment (start 78.943212 45.923212) (end 77.724 45.923212) (width 0.4064) (layer B.Cu) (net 14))
 (segment (start 81.788 45.078512) (end 80.9433 45.923212) (width 0.4064) (layer B.Cu) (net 14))
 (segment (start 80.9433 45.923212) (end 78.943212 45.923212) (width 0.4064) (layer B.Cu) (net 14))
 (segment (start 68.58 29.21) (end 73.406 34.036) (width 0.4064) (layer B.Cu) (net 18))
 (segment (start 73.406 34.036) (end 74.337276 34.036) (width 0.4064) (layer B.Cu) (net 18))
 (segment (start 74.337276 34.036) (end 77.207488 36.906212) (width 0.4064) (layer B.Cu) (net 18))
 (segment (start 77.207488 38.345488) (end 78.232 39.37) (width 0.4064) (layer B.Cu) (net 18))
 (segment (start 77.207488 36.906212) (end 77.207488 38.345488) (width 0.4064) (layer B.Cu) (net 18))
 (segment (start 78.232 39.37) (end 80.01 39.37) (width 0.4064) (layer B.Cu) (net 18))
 (segment (start 80.01 39.37) (end 80.1624 39.37) (width 0.4064) (layer B.Cu) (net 18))
 (segment (start 66.04 36.83) (end 66.04 37.973) (width 0.4064) (layer B.Cu) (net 12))
 (segment (start 66.04 37.973) (end 67.31 39.243) (width 0.4064) (layer B.Cu) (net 12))
 (via (at 67.31 39.243) (size 1.1176) (drill 0.4064) (layers F.Cu B.Cu) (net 12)))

